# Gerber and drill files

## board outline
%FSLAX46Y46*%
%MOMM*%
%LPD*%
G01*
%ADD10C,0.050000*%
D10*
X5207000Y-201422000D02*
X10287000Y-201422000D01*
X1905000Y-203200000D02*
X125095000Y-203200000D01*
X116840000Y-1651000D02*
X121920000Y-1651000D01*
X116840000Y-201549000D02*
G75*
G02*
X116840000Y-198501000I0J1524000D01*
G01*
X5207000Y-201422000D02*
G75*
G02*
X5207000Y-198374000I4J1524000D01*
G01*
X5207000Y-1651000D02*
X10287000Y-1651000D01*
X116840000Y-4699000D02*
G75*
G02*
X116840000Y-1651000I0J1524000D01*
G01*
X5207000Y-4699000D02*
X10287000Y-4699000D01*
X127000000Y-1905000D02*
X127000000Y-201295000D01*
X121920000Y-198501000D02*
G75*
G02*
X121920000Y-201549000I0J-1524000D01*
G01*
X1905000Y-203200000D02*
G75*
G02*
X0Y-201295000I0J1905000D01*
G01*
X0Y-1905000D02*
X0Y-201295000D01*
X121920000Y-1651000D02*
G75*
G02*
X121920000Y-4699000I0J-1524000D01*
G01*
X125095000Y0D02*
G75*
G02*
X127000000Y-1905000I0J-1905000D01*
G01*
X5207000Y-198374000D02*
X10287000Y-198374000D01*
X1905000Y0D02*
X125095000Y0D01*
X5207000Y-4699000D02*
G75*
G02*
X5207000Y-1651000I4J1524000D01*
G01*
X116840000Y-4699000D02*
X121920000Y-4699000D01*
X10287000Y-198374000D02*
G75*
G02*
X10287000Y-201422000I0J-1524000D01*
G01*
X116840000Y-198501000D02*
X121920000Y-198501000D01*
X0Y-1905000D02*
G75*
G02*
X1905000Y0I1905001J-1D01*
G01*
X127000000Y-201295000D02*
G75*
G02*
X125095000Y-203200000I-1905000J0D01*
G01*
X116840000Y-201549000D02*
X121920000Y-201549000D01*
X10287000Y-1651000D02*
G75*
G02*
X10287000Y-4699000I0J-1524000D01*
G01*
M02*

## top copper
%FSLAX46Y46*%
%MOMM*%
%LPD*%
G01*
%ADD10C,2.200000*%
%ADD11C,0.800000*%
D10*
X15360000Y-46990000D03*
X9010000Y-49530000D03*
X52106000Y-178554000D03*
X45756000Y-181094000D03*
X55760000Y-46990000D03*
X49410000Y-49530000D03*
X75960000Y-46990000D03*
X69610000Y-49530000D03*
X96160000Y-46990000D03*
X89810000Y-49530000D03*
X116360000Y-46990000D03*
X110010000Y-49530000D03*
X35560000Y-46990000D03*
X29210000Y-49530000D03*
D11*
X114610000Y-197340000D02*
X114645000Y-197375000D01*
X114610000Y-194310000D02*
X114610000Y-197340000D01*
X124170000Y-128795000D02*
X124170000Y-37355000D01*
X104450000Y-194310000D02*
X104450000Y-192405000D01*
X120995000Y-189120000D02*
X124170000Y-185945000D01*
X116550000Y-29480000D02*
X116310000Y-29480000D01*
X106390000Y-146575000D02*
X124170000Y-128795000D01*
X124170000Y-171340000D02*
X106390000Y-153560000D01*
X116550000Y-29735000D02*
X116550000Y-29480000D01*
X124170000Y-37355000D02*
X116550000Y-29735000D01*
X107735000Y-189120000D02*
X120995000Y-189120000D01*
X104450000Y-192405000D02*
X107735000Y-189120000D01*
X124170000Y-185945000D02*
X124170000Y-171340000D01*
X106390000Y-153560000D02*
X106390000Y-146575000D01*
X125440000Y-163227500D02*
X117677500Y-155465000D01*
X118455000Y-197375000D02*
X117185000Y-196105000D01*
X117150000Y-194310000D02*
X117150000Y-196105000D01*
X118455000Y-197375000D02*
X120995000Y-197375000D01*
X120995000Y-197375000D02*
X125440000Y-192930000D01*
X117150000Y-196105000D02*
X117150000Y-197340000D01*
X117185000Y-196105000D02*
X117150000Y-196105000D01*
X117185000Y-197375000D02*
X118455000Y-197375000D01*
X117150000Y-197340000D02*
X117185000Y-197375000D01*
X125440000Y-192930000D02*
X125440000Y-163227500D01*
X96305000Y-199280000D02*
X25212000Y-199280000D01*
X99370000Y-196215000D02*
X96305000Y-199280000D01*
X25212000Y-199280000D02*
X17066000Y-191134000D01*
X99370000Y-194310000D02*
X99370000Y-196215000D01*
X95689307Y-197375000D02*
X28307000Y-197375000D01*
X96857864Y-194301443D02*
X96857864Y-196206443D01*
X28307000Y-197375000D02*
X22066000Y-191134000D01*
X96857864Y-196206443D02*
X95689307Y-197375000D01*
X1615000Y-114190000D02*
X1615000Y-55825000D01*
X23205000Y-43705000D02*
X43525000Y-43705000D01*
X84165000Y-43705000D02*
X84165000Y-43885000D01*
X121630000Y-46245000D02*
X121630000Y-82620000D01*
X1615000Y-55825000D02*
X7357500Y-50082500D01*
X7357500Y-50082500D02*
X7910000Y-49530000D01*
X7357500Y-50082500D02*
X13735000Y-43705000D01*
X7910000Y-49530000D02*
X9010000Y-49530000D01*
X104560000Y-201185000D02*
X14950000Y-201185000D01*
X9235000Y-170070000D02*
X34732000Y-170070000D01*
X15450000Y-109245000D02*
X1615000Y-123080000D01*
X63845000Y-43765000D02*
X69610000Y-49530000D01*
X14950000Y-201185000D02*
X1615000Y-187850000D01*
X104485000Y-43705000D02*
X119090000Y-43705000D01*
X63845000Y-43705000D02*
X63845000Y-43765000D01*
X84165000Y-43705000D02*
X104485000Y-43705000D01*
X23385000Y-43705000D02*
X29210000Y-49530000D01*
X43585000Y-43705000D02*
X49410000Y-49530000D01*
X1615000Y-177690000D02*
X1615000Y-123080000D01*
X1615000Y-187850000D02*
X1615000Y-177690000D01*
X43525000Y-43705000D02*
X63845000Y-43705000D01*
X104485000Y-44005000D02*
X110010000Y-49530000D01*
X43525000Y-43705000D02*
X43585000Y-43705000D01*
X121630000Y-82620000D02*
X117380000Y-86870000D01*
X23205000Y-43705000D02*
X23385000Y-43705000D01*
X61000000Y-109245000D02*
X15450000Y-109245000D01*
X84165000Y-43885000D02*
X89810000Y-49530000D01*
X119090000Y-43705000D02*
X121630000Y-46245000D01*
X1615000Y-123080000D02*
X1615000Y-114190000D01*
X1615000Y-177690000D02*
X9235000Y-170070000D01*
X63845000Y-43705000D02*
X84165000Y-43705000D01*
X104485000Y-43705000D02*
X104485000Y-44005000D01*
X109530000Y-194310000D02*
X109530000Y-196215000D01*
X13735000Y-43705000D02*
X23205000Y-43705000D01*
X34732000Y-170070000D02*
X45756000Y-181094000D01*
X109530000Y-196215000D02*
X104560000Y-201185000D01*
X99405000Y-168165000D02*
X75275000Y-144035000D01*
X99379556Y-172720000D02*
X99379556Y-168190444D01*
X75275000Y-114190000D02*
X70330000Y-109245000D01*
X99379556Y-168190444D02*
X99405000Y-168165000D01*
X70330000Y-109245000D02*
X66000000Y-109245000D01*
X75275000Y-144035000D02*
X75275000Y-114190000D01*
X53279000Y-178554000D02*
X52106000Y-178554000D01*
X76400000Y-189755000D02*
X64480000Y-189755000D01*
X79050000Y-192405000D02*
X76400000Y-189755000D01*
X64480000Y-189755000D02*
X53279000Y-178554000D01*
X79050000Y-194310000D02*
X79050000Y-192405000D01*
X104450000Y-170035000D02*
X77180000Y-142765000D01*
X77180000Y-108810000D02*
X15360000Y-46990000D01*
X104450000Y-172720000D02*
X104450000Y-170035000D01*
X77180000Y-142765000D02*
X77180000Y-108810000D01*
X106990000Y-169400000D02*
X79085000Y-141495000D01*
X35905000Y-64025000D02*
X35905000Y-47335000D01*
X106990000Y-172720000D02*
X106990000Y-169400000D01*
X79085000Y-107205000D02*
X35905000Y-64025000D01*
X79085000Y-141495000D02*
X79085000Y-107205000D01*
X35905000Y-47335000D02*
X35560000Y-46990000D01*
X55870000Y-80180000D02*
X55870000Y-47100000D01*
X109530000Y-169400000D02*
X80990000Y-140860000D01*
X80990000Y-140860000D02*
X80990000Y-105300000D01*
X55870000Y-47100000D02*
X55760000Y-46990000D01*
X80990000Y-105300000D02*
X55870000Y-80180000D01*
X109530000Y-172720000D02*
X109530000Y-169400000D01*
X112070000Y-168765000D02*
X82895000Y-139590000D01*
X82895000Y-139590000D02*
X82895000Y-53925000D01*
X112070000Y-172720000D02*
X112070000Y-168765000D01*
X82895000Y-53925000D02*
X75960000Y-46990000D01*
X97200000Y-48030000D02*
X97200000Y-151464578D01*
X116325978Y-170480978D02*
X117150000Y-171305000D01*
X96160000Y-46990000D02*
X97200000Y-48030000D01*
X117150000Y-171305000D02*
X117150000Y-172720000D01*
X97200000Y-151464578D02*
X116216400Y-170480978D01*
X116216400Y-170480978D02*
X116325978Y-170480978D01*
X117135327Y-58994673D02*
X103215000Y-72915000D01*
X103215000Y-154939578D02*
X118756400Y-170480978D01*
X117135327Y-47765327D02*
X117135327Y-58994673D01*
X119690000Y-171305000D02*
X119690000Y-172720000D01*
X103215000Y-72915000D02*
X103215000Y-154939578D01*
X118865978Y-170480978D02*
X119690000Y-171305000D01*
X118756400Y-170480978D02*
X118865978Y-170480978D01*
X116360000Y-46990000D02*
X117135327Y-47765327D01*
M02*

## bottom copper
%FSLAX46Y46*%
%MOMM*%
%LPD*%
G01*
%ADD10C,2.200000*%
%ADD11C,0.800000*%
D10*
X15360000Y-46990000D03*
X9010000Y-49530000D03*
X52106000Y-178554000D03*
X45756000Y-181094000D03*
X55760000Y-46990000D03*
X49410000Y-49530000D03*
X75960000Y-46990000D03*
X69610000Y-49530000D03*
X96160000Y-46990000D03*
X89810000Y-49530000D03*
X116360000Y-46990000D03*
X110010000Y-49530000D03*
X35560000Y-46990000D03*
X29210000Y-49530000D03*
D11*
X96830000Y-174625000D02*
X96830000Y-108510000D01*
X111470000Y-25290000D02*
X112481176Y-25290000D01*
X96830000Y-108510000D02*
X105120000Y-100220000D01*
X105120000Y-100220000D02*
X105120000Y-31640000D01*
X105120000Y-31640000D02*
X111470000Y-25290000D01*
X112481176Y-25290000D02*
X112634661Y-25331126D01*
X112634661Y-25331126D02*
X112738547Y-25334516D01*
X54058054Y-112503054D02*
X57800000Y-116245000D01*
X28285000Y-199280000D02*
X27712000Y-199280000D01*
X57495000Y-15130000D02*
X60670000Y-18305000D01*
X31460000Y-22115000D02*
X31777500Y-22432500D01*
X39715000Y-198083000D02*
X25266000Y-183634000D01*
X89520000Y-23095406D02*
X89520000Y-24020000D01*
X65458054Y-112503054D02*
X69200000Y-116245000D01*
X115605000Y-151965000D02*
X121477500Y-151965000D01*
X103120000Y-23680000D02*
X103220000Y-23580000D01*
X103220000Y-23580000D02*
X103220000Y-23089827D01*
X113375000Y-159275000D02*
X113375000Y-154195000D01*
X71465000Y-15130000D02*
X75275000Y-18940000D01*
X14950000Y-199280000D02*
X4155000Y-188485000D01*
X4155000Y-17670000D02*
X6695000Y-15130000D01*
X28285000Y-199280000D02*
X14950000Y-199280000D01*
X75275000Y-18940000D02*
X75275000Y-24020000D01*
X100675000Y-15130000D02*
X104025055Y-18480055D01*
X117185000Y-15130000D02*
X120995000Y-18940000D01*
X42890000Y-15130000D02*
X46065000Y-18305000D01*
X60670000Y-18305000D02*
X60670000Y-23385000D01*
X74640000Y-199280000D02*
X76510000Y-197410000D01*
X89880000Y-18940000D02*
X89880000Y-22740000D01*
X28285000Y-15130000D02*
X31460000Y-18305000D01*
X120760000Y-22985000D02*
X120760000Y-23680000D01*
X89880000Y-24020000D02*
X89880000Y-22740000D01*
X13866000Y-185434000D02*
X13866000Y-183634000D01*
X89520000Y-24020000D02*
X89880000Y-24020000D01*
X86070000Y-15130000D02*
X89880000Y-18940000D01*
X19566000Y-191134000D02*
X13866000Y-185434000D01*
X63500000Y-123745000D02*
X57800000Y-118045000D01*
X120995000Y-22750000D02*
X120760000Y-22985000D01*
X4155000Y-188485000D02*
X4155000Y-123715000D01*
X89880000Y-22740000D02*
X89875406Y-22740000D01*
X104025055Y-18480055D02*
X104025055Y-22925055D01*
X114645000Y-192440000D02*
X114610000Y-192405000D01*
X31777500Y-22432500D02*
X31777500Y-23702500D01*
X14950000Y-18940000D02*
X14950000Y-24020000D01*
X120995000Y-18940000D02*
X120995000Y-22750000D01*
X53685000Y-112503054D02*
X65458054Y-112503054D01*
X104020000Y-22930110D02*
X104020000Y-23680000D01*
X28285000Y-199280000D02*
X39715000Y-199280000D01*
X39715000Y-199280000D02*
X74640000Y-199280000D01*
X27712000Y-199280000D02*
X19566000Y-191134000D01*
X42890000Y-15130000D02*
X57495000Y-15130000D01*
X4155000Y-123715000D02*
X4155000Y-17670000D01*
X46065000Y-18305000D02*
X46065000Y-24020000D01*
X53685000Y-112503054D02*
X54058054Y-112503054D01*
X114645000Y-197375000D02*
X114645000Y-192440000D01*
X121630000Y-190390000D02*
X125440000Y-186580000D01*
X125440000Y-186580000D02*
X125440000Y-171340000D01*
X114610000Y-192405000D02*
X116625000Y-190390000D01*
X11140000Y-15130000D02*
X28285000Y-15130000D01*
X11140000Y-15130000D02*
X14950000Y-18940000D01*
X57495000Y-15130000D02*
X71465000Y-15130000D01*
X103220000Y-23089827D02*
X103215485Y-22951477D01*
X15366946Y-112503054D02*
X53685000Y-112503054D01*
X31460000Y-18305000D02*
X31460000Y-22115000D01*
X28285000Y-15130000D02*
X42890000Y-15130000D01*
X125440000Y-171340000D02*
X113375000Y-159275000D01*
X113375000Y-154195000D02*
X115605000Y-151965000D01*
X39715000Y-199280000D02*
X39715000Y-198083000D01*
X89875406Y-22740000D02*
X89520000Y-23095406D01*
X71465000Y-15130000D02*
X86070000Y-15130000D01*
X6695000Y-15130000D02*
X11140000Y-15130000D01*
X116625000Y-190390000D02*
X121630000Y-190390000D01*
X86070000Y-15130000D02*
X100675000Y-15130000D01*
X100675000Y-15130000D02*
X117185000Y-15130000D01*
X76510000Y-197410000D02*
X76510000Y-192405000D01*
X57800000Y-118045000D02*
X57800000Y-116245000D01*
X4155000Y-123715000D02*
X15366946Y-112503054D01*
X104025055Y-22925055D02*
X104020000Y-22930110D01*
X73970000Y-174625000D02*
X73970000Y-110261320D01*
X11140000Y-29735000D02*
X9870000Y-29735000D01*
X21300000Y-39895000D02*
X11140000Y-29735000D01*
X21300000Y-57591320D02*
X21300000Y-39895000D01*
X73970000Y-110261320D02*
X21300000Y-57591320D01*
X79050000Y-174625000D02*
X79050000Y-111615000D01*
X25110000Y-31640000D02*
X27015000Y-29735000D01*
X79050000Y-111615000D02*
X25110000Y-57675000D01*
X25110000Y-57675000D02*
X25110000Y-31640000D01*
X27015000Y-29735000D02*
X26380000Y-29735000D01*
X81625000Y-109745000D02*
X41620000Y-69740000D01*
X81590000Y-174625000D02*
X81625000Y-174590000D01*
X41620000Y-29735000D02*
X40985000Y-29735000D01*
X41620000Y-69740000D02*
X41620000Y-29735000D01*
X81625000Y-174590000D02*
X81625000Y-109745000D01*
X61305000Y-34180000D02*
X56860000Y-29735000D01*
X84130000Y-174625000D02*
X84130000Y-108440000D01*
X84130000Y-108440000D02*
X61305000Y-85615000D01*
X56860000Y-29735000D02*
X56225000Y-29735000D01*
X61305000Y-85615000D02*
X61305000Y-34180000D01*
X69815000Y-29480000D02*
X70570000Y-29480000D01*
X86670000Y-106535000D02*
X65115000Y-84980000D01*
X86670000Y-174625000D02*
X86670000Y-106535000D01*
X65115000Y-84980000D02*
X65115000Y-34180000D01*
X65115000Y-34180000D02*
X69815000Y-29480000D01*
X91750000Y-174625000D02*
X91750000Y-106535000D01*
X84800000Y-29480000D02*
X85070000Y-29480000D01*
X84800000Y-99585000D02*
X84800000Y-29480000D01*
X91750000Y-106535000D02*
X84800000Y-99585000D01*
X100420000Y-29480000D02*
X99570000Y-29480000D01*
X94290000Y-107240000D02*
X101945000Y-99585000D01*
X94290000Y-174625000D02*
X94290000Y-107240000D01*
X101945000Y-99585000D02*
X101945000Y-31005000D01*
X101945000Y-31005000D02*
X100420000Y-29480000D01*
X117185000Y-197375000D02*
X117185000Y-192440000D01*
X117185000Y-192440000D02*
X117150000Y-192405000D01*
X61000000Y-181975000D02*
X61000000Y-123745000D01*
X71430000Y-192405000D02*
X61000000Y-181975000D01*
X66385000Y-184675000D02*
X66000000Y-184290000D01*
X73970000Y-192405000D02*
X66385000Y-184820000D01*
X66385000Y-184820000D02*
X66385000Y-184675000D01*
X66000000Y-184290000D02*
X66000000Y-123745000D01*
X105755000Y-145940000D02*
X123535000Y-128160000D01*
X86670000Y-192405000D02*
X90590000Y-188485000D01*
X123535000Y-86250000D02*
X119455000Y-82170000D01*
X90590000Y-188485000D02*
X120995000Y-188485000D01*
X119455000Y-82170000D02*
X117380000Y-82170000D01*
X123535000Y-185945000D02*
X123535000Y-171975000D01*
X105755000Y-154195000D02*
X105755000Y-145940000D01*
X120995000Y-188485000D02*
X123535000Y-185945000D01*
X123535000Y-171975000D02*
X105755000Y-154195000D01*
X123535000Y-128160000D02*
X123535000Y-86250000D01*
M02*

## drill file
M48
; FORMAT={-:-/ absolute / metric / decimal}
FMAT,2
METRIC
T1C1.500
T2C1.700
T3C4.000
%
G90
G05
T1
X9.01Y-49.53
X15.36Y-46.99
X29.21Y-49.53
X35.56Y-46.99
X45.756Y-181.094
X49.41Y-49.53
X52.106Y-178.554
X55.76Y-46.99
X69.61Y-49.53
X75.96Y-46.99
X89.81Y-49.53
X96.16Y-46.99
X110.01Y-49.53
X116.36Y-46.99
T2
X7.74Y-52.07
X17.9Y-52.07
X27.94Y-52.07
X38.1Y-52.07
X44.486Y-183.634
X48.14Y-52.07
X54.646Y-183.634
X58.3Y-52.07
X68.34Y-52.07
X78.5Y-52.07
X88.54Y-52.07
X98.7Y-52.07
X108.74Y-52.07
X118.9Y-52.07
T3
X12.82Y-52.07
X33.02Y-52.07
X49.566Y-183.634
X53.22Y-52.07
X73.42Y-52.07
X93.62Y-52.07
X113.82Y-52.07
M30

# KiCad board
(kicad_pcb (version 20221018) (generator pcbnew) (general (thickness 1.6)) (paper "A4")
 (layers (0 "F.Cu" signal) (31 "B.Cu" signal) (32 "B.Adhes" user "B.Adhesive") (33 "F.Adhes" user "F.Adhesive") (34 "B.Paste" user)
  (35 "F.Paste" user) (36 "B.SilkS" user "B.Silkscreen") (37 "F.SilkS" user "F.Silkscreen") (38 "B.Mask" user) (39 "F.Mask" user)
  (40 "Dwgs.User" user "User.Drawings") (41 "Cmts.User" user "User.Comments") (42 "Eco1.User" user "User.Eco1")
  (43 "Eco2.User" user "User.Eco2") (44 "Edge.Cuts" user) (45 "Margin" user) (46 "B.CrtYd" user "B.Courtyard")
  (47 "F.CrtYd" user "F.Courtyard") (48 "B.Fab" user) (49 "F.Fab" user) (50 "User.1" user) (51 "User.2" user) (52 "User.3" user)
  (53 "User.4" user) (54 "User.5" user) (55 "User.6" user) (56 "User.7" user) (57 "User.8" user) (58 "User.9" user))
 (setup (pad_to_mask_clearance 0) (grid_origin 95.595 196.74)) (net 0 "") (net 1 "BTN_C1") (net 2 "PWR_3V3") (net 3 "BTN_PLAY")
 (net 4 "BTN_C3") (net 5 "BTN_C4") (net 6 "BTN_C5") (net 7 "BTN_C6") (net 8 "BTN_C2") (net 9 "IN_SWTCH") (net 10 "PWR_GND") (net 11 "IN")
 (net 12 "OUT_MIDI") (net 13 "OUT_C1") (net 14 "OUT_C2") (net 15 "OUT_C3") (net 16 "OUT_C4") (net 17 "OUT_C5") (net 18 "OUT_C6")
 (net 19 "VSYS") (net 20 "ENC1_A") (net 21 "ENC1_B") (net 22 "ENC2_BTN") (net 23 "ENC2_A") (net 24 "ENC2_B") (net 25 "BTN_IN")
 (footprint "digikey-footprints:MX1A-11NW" (layer "F.Cu") (at 11.55 42.545)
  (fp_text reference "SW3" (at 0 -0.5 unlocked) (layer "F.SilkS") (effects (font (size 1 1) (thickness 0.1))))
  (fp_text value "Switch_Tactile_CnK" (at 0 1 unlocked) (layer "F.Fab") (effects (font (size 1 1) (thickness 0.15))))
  (pad "" np_thru_hole circle (at -3.81 9.525) (size 1.7 1.7) (drill 1.7) (layers "*.Cu" "*.Mask"))
  (pad "" np_thru_hole circle (at 1.27 9.525) (size 4 4) (drill 4) (layers "*.Cu" "*.Mask"))
  (pad "" np_thru_hole circle (at 6.35 9.525) (size 1.7 1.7) (drill 1.7) (layers "*.Cu" "*.Mask"))
  (pad "1" thru_hole circle (at 3.81 4.445) (size 2.2 2.2) (drill 1.5) (layers "*.Cu" "*.Mask") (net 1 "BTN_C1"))
  (pad "2" thru_hole circle (at -2.54 6.985) (size 2.2 2.2) (drill 1.5) (layers "*.Cu" "*.Mask") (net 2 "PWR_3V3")))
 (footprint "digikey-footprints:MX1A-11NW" (layer "F.Cu") (at 48.296 174.109)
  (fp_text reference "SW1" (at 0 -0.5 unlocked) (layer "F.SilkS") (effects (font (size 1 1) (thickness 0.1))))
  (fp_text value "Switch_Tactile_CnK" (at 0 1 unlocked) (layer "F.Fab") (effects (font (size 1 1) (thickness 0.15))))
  (pad "" np_thru_hole circle (at -3.81 9.525) (size 1.7 1.7) (drill 1.7) (layers "*.Cu" "*.Mask"))
  (pad "" np_thru_hole circle (at 1.27 9.525) (size 4 4) (drill 4) (layers "*.Cu" "*.Mask"))
  (pad "" np_thru_hole circle (at 6.35 9.525) (size 1.7 1.7) (drill 1.7) (layers "*.Cu" "*.Mask"))
  (pad "1" thru_hole circle (at 3.81 4.445) (size 2.2 2.2) (drill 1.5) (layers "*.Cu" "*.Mask") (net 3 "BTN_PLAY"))
  (pad "2" thru_hole circle (at -2.54 6.985) (size 2.2 2.2) (drill 1.5) (layers "*.Cu" "*.Mask") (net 2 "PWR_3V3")))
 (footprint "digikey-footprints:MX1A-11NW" (layer "F.Cu") (at 51.95 42.545)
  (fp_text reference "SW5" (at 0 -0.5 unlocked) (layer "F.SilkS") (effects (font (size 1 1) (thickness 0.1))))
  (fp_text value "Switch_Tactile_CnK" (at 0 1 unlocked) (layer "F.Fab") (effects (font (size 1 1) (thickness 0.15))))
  (pad "" np_thru_hole circle (at -3.81 9.525) (size 1.7 1.7) (drill 1.7) (layers "*.Cu" "*.Mask"))
  (pad "" np_thru_hole circle (at 1.27 9.525) (size 4 4) (drill 4) (layers "*.Cu" "*.Mask"))
  (pad "" np_thru_hole circle (at 6.35 9.525) (size 1.7 1.7) (drill 1.7) (layers "*.Cu" "*.Mask"))
  (pad "1" thru_hole circle (at 3.81 4.445) (size 2.2 2.2) (drill 1.5) (layers "*.Cu" "*.Mask") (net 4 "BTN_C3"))
  (pad "2" thru_hole circle (at -2.54 6.985) (size 2.2 2.2) (drill 1.5) (layers "*.Cu" "*.Mask") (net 2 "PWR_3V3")))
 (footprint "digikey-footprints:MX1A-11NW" (layer "F.Cu") (at 72.15 42.545)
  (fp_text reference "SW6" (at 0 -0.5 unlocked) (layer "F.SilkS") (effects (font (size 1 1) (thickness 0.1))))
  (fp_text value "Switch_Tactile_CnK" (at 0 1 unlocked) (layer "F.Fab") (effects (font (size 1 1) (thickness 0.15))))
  (pad "" np_thru_hole circle (at -3.81 9.525) (size 1.7 1.7) (drill 1.7) (layers "*.Cu" "*.Mask"))
  (pad "" np_thru_hole circle (at 1.27 9.525) (size 4 4) (drill 4) (layers "*.Cu" "*.Mask"))
  (pad "" np_thru_hole circle (at 6.35 9.525) (size 1.7 1.7) (drill 1.7) (layers "*.Cu" "*.Mask"))
  (pad "1" thru_hole circle (at 3.81 4.445) (size 2.2 2.2) (drill 1.5) (layers "*.Cu" "*.Mask") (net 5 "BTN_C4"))
  (pad "2" thru_hole circle (at -2.54 6.985) (size 2.2 2.2) (drill 1.5) (layers "*.Cu" "*.Mask") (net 2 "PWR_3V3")))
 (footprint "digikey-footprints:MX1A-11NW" (layer "F.Cu") (at 92.35 42.545)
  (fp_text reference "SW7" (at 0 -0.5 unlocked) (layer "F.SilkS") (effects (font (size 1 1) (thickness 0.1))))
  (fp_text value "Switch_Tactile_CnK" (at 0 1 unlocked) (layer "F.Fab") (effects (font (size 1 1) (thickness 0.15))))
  (pad "" np_thru_hole circle (at -3.81 9.525) (size 1.7 1.7) (drill 1.7) (layers "*.Cu" "*.Mask"))
  (pad "" np_thru_hole circle (at 1.27 9.525) (size 4 4) (drill 4) (layers "*.Cu" "*.Mask"))
  (pad "" np_thru_hole circle (at 6.35 9.525) (size 1.7 1.7) (drill 1.7) (layers "*.Cu" "*.Mask"))
  (pad "1" thru_hole circle (at 3.81 4.445) (size 2.2 2.2) (drill 1.5) (layers "*.Cu" "*.Mask") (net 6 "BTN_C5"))
  (pad "2" thru_hole circle (at -2.54 6.985) (size 2.2 2.2) (drill 1.5) (layers "*.Cu" "*.Mask") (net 2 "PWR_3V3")))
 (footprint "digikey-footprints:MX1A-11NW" (layer "F.Cu") (at 112.55 42.545)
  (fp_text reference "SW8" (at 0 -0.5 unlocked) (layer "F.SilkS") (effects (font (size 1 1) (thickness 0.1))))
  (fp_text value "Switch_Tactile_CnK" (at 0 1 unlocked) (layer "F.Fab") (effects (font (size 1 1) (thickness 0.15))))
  (pad "" np_thru_hole circle (at -3.81 9.525) (size 1.7 1.7) (drill 1.7) (layers "*.Cu" "*.Mask"))
  (pad "" np_thru_hole circle (at 1.27 9.525) (size 4 4) (drill 4) (layers "*.Cu" "*.Mask"))
  (pad "" np_thru_hole circle (at 6.35 9.525) (size 1.7 1.7) (drill 1.7) (layers "*.Cu" "*.Mask"))
  (pad "1" thru_hole circle (at 3.81 4.445) (size 2.2 2.2) (drill 1.5) (layers "*.Cu" "*.Mask") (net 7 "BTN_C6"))
  (pad "2" thru_hole circle (at -2.54 6.985) (size 2.2 2.2) (drill 1.5) (layers "*.Cu" "*.Mask") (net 2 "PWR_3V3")))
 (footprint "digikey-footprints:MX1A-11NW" (layer "F.Cu") (at 31.75 42.545)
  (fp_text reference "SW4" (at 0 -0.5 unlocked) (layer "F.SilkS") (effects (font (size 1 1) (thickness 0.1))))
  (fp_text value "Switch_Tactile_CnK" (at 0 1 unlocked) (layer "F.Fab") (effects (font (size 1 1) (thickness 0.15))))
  (pad "" np_thru_hole circle (at -3.81 9.525) (size 1.7 1.7) (drill 1.7) (layers "*.Cu" "*.Mask"))
  (pad "" np_thru_hole circle (at 1.27 9.525) (size 4 4) (drill 4) (layers "*.Cu" "*.Mask"))
  (pad "" np_thru_hole circle (at 6.35 9.525) (size 1.7 1.7) (drill 1.7) (layers "*.Cu" "*.Mask"))
  (pad "1" thru_hole circle (at 3.81 4.445) (size 2.2 2.2) (drill 1.5) (layers "*.Cu" "*.Mask") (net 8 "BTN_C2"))
  (pad "2" thru_hole circle (at -2.54 6.985) (size 2.2 2.2) (drill 1.5) (layers "*.Cu" "*.Mask") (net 2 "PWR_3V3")))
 (gr_line (start 5.207 201.422) (end 10.287 201.422) (stroke (width 0.05) (type solid)) (layer "Edge.Cuts"))
 (gr_line (start 1.905 203.2) (end 125.095 203.2) (stroke (width 0.05) (type default)) (layer "Edge.Cuts"))
 (gr_line (start 116.84 1.651) (end 121.92 1.651) (stroke (width 0.05) (type solid)) (layer "Edge.Cuts"))
 (gr_arc (start 116.84 201.549) (mid 115.316004 200.025002) (end 116.84 198.501) (stroke (width 0.05) (type solid)) (layer "Edge.Cuts"))
 (gr_arc (start 5.207 201.422) (mid 3.683004 199.898002) (end 5.207 198.374) (stroke (width 0.05) (type solid)) (layer "Edge.Cuts"))
 (gr_line (start 5.207 1.651) (end 10.287 1.651) (stroke (width 0.05) (type solid)) (layer "Edge.Cuts"))
 (gr_arc (start 116.84 4.699) (mid 115.316004 3.175002) (end 116.84 1.651) (stroke (width 0.05) (type solid)) (layer "Edge.Cuts"))
 (gr_line (start 5.207 4.699) (end 10.287 4.699) (stroke (width 0.05) (type solid)) (layer "Edge.Cuts"))
 (gr_line (start 127 1.905) (end 127 201.295) (stroke (width 0.05) (type default)) (layer "Edge.Cuts"))
 (gr_arc (start 121.92 198.501) (mid 123.444004 200.025002) (end 121.92 201.549) (stroke (width 0.05) (type solid)) (layer "Edge.Cuts"))
 (gr_arc (start 1.905 203.2) (mid 0.557962 202.642038) (end 0 201.295) (stroke (width 0.05) (type solid)) (layer "Edge.Cuts"))
 (gr_line (start 0 1.905) (end 0 201.295) (stroke (width 0.05) (type default)) (layer "Edge.Cuts"))
 (gr_arc (start 121.92 1.651) (mid 123.444004 3.175002) (end 121.92 4.699) (stroke (width 0.05) (type solid)) (layer "Edge.Cuts"))
 (gr_arc (start 125.095 0) (mid 126.442038 0.557962) (end 127 1.905) (stroke (width 0.05) (type solid)) (layer "Edge.Cuts"))
 (gr_line (start 5.207 198.374) (end 10.287 198.374) (stroke (width 0.05) (type solid)) (layer "Edge.Cuts"))
 (gr_line (start 1.905 0) (end 125.095 0) (stroke (width 0.05) (type default)) (layer "Edge.Cuts"))
 (gr_arc (start 5.207 4.699) (mid 3.683004 3.175002) (end 5.207 1.651) (stroke (width 0.05) (type solid)) (layer "Edge.Cuts"))
 (gr_line (start 116.84 4.699) (end 121.92 4.699) (stroke (width 0.05) (type solid)) (layer "Edge.Cuts"))
 (gr_arc (start 10.287 198.374) (mid 11.811004 199.898002) (end 10.287 201.422) (stroke (width 0.05) (type solid)) (layer "Edge.Cuts"))
 (gr_line (start 116.84 198.501) (end 121.92 198.501) (stroke (width 0.05) (type solid)) (layer "Edge.Cuts"))
 (gr_arc (start 0 1.905) (mid 0.557962 0.557962) (end 1.905 0) (stroke (width 0.05) (type solid)) (layer "Edge.Cuts"))
 (gr_arc (start 127 201.295) (mid 126.442038 202.642038) (end 125.095 203.2) (stroke (width 0.05) (type solid)) (layer "Edge.Cuts"))
 (gr_line (start 116.84 201.549) (end 121.92 201.549) (stroke (width 0.05) (type solid)) (layer "Edge.Cuts"))
 (gr_arc (start 10.287 1.651) (mid 11.811004 3.175002) (end 10.287 4.699) (stroke (width 0.05) (type solid)) (layer "Edge.Cuts"))
 (segment (start 96.83 174.625) (end 96.83 108.51) (width 0.8) (layer "B.Cu") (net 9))
 (segment (start 111.47 25.29) (end 112.481176 25.29) (width 0.8) (layer "B.Cu") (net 9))
 (segment (start 96.83 108.51) (end 105.12 100.22) (width 0.8) (layer "B.Cu") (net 9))
 (segment (start 105.12 100.22) (end 105.12 31.64) (width 0.8) (layer "B.Cu") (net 9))
 (segment (start 105.12 31.64) (end 111.47 25.29) (width 0.8) (layer "B.Cu") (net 9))
 (segment (start 112.481176 25.29) (end 112.634661 25.331126) (width 0.8) (layer "B.Cu") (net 9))
 (segment (start 112.634661 25.331126) (end 112.738547 25.334516) (width 0.8) (layer "B.Cu") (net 9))
 (segment (start 114.61 197.34) (end 114.645 197.375) (width 0.8) (layer "F.Cu") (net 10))
 (segment (start 114.61 194.31) (end 114.61 197.34) (width 0.8) (layer "F.Cu") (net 10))
 (segment (start 54.058054 112.503054) (end 57.8 116.245) (width 0.8) (layer "B.Cu") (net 10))
 (segment (start 28.285 199.28) (end 27.712 199.28) (width 0.8) (layer "B.Cu") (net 10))
 (segment (start 57.495 15.13) (end 60.67 18.305) (width 0.8) (layer "B.Cu") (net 10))
 (segment (start 31.46 22.115) (end 31.7775 22.4325) (width 0.8) (layer "B.Cu") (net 10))
 (segment (start 39.715 198.083) (end 25.266 183.634) (width 0.8) (layer "B.Cu") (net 10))
 (segment (start 89.52 23.095406) (end 89.52 24.02) (width 0.8) (layer "B.Cu") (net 10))
 (segment (start 65.458054 112.503054) (end 69.2 116.245) (width 0.8) (layer "B.Cu") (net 10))
 (segment (start 115.605 151.965) (end 121.4775 151.965) (width 0.8) (layer "B.Cu") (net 10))
 (segment (start 103.12 23.68) (end 103.22 23.58) (width 0.8) (layer "B.Cu") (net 10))
 (segment (start 103.22 23.58) (end 103.22 23.089827) (width 0.8) (layer "B.Cu") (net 10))
 (segment (start 113.375 159.275) (end 113.375 154.195) (width 0.8) (layer "B.Cu") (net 10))
 (segment (start 71.465 15.13) (end 75.275 18.94) (width 0.8) (layer "B.Cu") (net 10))
 (segment (start 14.95 199.28) (end 4.155 188.485) (width 0.8) (layer "B.Cu") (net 10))
 (segment (start 4.155 17.67) (end 6.695 15.13) (width 0.8) (layer "B.Cu") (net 10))
 (segment (start 28.285 199.28) (end 14.95 199.28) (width 0.8) (layer "B.Cu") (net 10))
 (segment (start 75.275 18.94) (end 75.275 24.02) (width 0.8) (layer "B.Cu") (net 10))
 (segment (start 100.675 15.13) (end 104.025055 18.480055) (width 0.8) (layer "B.Cu") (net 10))
 (segment (start 117.185 15.13) (end 120.995 18.94) (width 0.8) (layer "B.Cu") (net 10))
 (segment (start 42.89 15.13) (end 46.065 18.305) (width 0.8) (layer "B.Cu") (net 10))
 (segment (start 60.67 18.305) (end 60.67 23.385) (width 0.8) (layer "B.Cu") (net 10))
 (segment (start 74.64 199.28) (end 76.51 197.41) (width 0.8) (layer "B.Cu") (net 10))
 (segment (start 89.88 18.94) (end 89.88 22.74) (width 0.8) (layer "B.Cu") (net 10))
 (segment (start 28.285 15.13) (end 31.46 18.305) (width 0.8) (layer "B.Cu") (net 10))
 (segment (start 120.76 22.985) (end 120.76 23.68) (width 0.8) (layer "B.Cu") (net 10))
 (segment (start 89.88 24.02) (end 89.88 22.74) (width 0.8) (layer "B.Cu") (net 10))
 (segment (start 13.866 185.434) (end 13.866 183.634) (width 0.8) (layer "B.Cu") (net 10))
 (segment (start 89.52 24.02) (end 89.88 24.02) (width 0.8) (layer "B.Cu") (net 10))
 (segment (start 86.07 15.13) (end 89.88 18.94) (width 0.8) (layer "B.Cu") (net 10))
 (segment (start 19.566 191.134) (end 13.866 185.434) (width 0.8) (layer "B.Cu") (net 10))
 (segment (start 63.5 123.745) (end 57.8 118.045) (width 0.8) (layer "B.Cu") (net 10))
 (segment (start 120.995 22.75) (end 120.76 22.985) (width 0.8) (layer "B.Cu") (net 10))
 (segment (start 4.155 188.485) (end 4.155 123.715) (width 0.8) (layer "B.Cu") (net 10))
 (segment (start 89.88 22.74) (end 89.875406 22.74) (width 0.8) (layer "B.Cu") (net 10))
 (segment (start 104.025055 18.480055) (end 104.025055 22.925055) (width 0.8) (layer "B.Cu") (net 10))
 (segment (start 114.645 192.44) (end 114.61 192.405) (width 0.8) (layer "B.Cu") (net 10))
 (segment (start 31.7775 22.4325) (end 31.7775 23.7025) (width 0.8) (layer "B.Cu") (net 10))
 (segment (start 14.95 18.94) (end 14.95 24.02) (width 0.8) (layer "B.Cu") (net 10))
 (segment (start 120.995 18.94) (end 120.995 22.75) (width 0.8) (layer "B.Cu") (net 10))
 (segment (start 53.685 112.503054) (end 65.458054 112.503054) (width 0.8) (layer "B.Cu") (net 10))
 (segment (start 104.02 22.93011) (end 104.02 23.68) (width 0.8) (layer "B.Cu") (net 10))
 (segment (start 28.285 199.28) (end 39.715 199.28) (width 0.8) (layer "B.Cu") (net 10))
 (segment (start 39.715 199.28) (end 74.64 199.28) (width 0.8) (layer "B.Cu") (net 10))
 (segment (start 27.712 199.28) (end 19.566 191.134) (width 0.8) (layer "B.Cu") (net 10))
 (segment (start 42.89 15.13) (end 57.495 15.13) (width 0.8) (layer "B.Cu") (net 10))
 (segment (start 4.155 123.715) (end 4.155 17.67) (width 0.8) (layer "B.Cu") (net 10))
 (segment (start 46.065 18.305) (end 46.065 24.02) (width 0.8) (layer "B.Cu") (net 10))
 (segment (start 53.685 112.503054) (end 54.058054 112.503054) (width 0.8) (layer "B.Cu") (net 10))
 (segment (start 114.645 197.375) (end 114.645 192.44) (width 0.8) (layer "B.Cu") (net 10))
 (segment (start 121.63 190.39) (end 125.44 186.58) (width 0.8) (layer "B.Cu") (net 10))
 (segment (start 125.44 186.58) (end 125.44 171.34) (width 0.8) (layer "B.Cu") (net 10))
 (segment (start 114.61 192.405) (end 116.625 190.39) (width 0.8) (layer "B.Cu") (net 10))
 (segment (start 11.14 15.13) (end 28.285 15.13) (width 0.8) (layer "B.Cu") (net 10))
 (segment (start 11.14 15.13) (end 14.95 18.94) (width 0.8) (layer "B.Cu") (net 10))
 (segment (start 57.495 15.13) (end 71.465 15.13) (width 0.8) (layer "B.Cu") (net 10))
 (segment (start 103.22 23.089827) (end 103.215485 22.951477) (width 0.8) (layer "B.Cu") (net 10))
 (segment (start 15.366946 112.503054) (end 53.685 112.503054) (width 0.8) (layer "B.Cu") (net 10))
 (segment (start 31.46 18.305) (end 31.46 22.115) (width 0.8) (layer "B.Cu") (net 10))
 (segment (start 28.285 15.13) (end 42.89 15.13) (width 0.8) (layer "B.Cu") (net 10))
 (segment (start 125.44 171.34) (end 113.375 159.275) (width 0.8) (layer "B.Cu") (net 10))
 (segment (start 113.375 154.195) (end 115.605 151.965) (width 0.8) (layer "B.Cu") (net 10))
 (segment (start 39.715 199.28) (end 39.715 198.083) (width 0.8) (layer "B.Cu") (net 10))
 (segment (start 89.875406 22.74) (end 89.52 23.095406) (width 0.8) (layer "B.Cu") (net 10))
 (segment (start 71.465 15.13) (end 86.07 15.13) (width 0.8) (layer "B.Cu") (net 10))
 (segment (start 6.695 15.13) (end 11.14 15.13) (width 0.8) (layer "B.Cu") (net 10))
 (segment (start 116.625 190.39) (end 121.63 190.39) (width 0.8) (layer "B.Cu") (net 10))
 (segment (start 86.07 15.13) (end 100.675 15.13) (width 0.8) (layer "B.Cu") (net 10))
 (segment (start 100.675 15.13) (end 117.185 15.13) (width 0.8) (layer "B.Cu") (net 10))
 (segment (start 76.51 197.41) (end 76.51 192.405) (width 0.8) (layer "B.Cu") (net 10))
 (segment (start 57.8 118.045) (end 57.8 116.245) (width 0.8) (layer "B.Cu") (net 10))
 (segment (start 4.155 123.715) (end 15.366946 112.503054) (width 0.8) (layer "B.Cu") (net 10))
 (segment (start 104.025055 22.925055) (end 104.02 22.93011) (width 0.8) (layer "B.Cu") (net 10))
 (segment (start 124.17 128.795) (end 124.17 37.355) (width 0.8) (layer "F.Cu") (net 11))
 (segment (start 104.45 194.31) (end 104.45 192.405) (width 0.8) (layer "F.Cu") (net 11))
 (segment (start 120.995 189.12) (end 124.17 185.945) (width 0.8) (layer "F.Cu") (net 11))
 (segment (start 116.55 29.48) (end 116.31 29.48) (width 0.8) (layer "F.Cu") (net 11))
 (segment (start 106.39 146.575) (end 124.17 128.795) (width 0.8) (layer "F.Cu") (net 11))
 (segment (start 124.17 171.34) (end 106.39 153.56) (width 0.8) (layer "F.Cu") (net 11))
 (segment (start 116.55 29.735) (end 116.55 29.48) (width 0.8) (layer "F.Cu") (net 11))
 (segment (start 124.17 37.355) (end 116.55 29.735) (width 0.8) (layer "F.Cu") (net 11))
 (segment (start 107.735 189.12) (end 120.995 189.12) (width 0.8) (layer "F.Cu") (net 11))
 (segment (start 104.45 192.405) (end 107.735 189.12) (width 0.8) (layer "F.Cu") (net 11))
 (segment (start 124.17 185.945) (end 124.17 171.34) (width 0.8) (layer "F.Cu") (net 11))
 (segment (start 106.39 153.56) (end 106.39 146.575) (width 0.8) (layer "F.Cu") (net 11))
 (segment (start 73.97 174.625) (end 73.97 110.26132) (width 0.8) (layer "B.Cu") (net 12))
 (segment (start 11.14 29.735) (end 9.87 29.735) (width 0.8) (layer "B.Cu") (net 12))
 (segment (start 21.3 39.895) (end 11.14 29.735) (width 0.8) (layer "B.Cu") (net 12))
 (segment (start 21.3 57.59132) (end 21.3 39.895) (width 0.8) (layer "B.Cu") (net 12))
 (segment (start 73.97 110.26132) (end 21.3 57.59132) (width 0.8) (layer "B.Cu") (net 12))
 (segment (start 79.05 174.625) (end 79.05 111.615) (width 0.8) (layer "B.Cu") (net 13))
 (segment (start 25.11 31.64) (end 27.015 29.735) (width 0.8) (layer "B.Cu") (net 13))
 (segment (start 79.05 111.615) (end 25.11 57.675) (width 0.8) (layer "B.Cu") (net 13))
 (segment (start 25.11 57.675) (end 25.11 31.64) (width 0.8) (layer "B.Cu") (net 13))
 (segment (start 27.015 29.735) (end 26.38 29.735) (width 0.8) (layer "B.Cu") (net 13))
 (segment (start 81.625 109.745) (end 41.62 69.74) (width 0.8) (layer "B.Cu") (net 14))
 (segment (start 81.59 174.625) (end 81.625 174.59) (width 0.8) (layer "B.Cu") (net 14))
 (segment (start 41.62 29.735) (end 40.985 29.735) (width 0.8) (layer "B.Cu") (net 14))
 (segment (start 41.62 69.74) (end 41.62 29.735) (width 0.8) (layer "B.Cu") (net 14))
 (segment (start 81.625 174.59) (end 81.625 109.745) (width 0.8) (layer "B.Cu") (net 14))
 (segment (start 61.305 34.18) (end 56.86 29.735) (width 0.8) (layer "B.Cu") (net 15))
 (segment (start 84.13 174.625) (end 84.13 108.44) (width 0.8) (layer "B.Cu") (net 15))
 (segment (start 84.13 108.44) (end 61.305 85.615) (width 0.8) (layer "B.Cu") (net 15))
 (segment (start 56.86 29.735) (end 56.225 29.735) (width 0.8) (layer "B.Cu") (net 15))
 (segment (start 61.305 85.615) (end 61.305 34.18) (width 0.8) (layer "B.Cu") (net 15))
 (segment (start 69.815 29.48) (end 70.57 29.48) (width 0.8) (layer "B.Cu") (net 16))
 (segment (start 86.67 106.535) (end 65.115 84.98) (width 0.8) (layer "B.Cu") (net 16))
 (segment (start 86.67 174.625) (end 86.67 106.535) (width 0.8) (layer "B.Cu") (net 16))
 (segment (start 65.115 84.98) (end 65.115 34.18) (width 0.8) (layer "B.Cu") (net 16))
 (segment (start 65.115 34.18) (end 69.815 29.48) (width 0.8) (layer "B.Cu") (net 16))
 (segment (start 91.75 174.625) (end 91.75 106.535) (width 0.8) (layer "B.Cu") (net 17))
 (segment (start 84.8 29.48) (end 85.07 29.48) (width 0.8) (layer "B.Cu") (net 17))
 (segment (start 84.8 99.585) (end 84.8 29.48) (width 0.8) (layer "B.Cu") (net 17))
 (segment (start 91.75 106.535) (end 84.8 99.585) (width 0.8) (layer "B.Cu") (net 17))
 (segment (start 100.42 29.48) (end 99.57 29.48) (width 0.8) (layer "B.Cu") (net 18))
 (segment (start 94.29 107.24) (end 101.945 99.585) (width 0.8) (layer "B.Cu") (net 18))
 (segment (start 94.29 174.625) (end 94.29 107.24) (width 0.8) (layer "B.Cu") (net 18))
 (segment (start 101.945 99.585) (end 101.945 31.005) (width 0.8) (layer "B.Cu") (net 18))
 (segment (start 101.945 31.005) (end 100.42 29.48) (width 0.8) (layer "B.Cu") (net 18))
 (segment (start 125.44 163.2275) (end 117.6775 155.465) (width 0.8) (layer "F.Cu") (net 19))
 (segment (start 118.455 197.375) (end 117.185 196.105) (width 0.8) (layer "F.Cu") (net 19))
 (segment (start 117.15 194.31) (end 117.15 196.105) (width 0.8) (layer "F.Cu") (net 19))
 (segment (start 118.455 197.375) (end 120.995 197.375) (width 0.8) (layer "F.Cu") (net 19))
 (segment (start 120.995 197.375) (end 125.44 192.93) (width 0.8) (layer "F.Cu") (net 19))
 (segment (start 117.15 196.105) (end 117.15 197.34) (width 0.8) (layer "F.Cu") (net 19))
 (segment (start 117.185 196.105) (end 117.15 196.105) (width 0.8) (layer "F.Cu") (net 19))
 (segment (start 117.185 197.375) (end 118.455 197.375) (width 0.8) (layer "F.Cu") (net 19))
 (segment (start 117.15 197.34) (end 117.185 197.375) (width 0.8) (layer "F.Cu") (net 19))
 (segment (start 125.44 192.93) (end 125.44 163.2275) (width 0.8) (layer "F.Cu") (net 19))
 (segment (start 117.185 197.375) (end 117.185 192.44) (width 0.8) (layer "B.Cu") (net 19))
 (segment (start 117.185 192.44) (end 117.15 192.405) (width 0.8) (layer "B.Cu") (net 19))
 (segment (start 96.305 199.28) (end 25.212 199.28) (width 0.8) (layer "F.Cu") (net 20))
 (segment (start 99.37 196.215) (end 96.305 199.28) (width 0.8) (layer "F.Cu") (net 20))
 (segment (start 25.212 199.28) (end 17.066 191.134) (width 0.8) (layer "F.Cu") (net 20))
 (segment (start 99.37 194.31) (end 99.37 196.215) (width 0.8) (layer "F.Cu") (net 20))
 (segment (start 95.689307 197.375) (end 28.307 197.375) (width 0.8) (layer "F.Cu") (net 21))
 (segment (start 96.857864 194.301443) (end 96.857864 196.206443) (width 0.8) (layer "F.Cu") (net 21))
 (segment (start 28.307 197.375) (end 22.066 191.134) (width 0.8) (layer "F.Cu") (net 21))
 (segment (start 96.857864 196.206443) (end 95.689307 197.375) (width 0.8) (layer "F.Cu") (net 21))
 (segment (start 1.615 114.19) (end 1.615 55.825) (width 0.8) (layer "F.Cu") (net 2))
 (segment (start 23.205 43.705) (end 43.525 43.705) (width 0.8) (layer "F.Cu") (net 2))
 (segment (start 84.165 43.705) (end 84.165 43.885) (width 0.8) (layer "F.Cu") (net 2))
 (segment (start 121.63 46.245) (end 121.63 82.62) (width 0.8) (layer "F.Cu") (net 2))
 (segment (start 1.615 55.825) (end 7.3575 50.0825) (width 0.8) (layer "F.Cu") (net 2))
 (segment (start 7.3575 50.0825) (end 7.91 49.53) (width 0.8) (layer "F.Cu") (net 2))
 (segment (start 7.3575 50.0825) (end 13.735 43.705) (width 0.8) (layer "F.Cu") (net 2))
 (segment (start 7.91 49.53) (end 9.01 49.53) (width 0.8) (layer "F.Cu") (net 2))
 (segment (start 104.56 201.185) (end 14.95 201.185) (width 0.8) (layer "F.Cu") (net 2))
 (segment (start 9.235 170.07) (end 34.732 170.07) (width 0.8) (layer "F.Cu") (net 2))
 (segment (start 15.45 109.245) (end 1.615 123.08) (width 0.8) (layer "F.Cu") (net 2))
 (segment (start 63.845 43.765) (end 69.61 49.53) (width 0.8) (layer "F.Cu") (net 2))
 (segment (start 14.95 201.185) (end 1.615 187.85) (width 0.8) (layer "F.Cu") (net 2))
 (segment (start 104.485 43.705) (end 119.09 43.705) (width 0.8) (layer "F.Cu") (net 2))
 (segment (start 63.845 43.705) (end 63.845 43.765) (width 0.8) (layer "F.Cu") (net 2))
 (segment (start 84.165 43.705) (end 104.485 43.705) (width 0.8) (layer "F.Cu") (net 2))
 (segment (start 23.385 43.705) (end 29.21 49.53) (width 0.8) (layer "F.Cu") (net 2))
 (segment (start 43.585 43.705) (end 49.41 49.53) (width 0.8) (layer "F.Cu") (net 2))
 (segment (start 1.615 177.69) (end 1.615 123.08) (width 0.8) (layer "F.Cu") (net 2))
 (segment (start 1.615 187.85) (end 1.615 177.69) (width 0.8) (layer "F.Cu") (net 2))
 (segment (start 43.525 43.705) (end 63.845 43.705) (width 0.8) (layer "F.Cu") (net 2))
 (segment (start 104.485 44.005) (end 110.01 49.53) (width 0.8) (layer "F.Cu") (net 2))
 (segment (start 43.525 43.705) (end 43.585 43.705) (width 0.8) (layer "F.Cu") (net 2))
 (segment (start 121.63 82.62) (end 117.38 86.87) (width 0.8) (layer "F.Cu") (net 2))
 (segment (start 23.205 43.705) (end 23.385 43.705) (width 0.8) (layer "F.Cu") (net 2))
 (segment (start 61 109.245) (end 15.45 109.245) (width 0.8) (layer "F.Cu") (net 2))
 (segment (start 84.165 43.885) (end 89.81 49.53) (width 0.8) (layer "F.Cu") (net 2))
 (segment (start 119.09 43.705) (end 121.63 46.245) (width 0.8) (layer "F.Cu") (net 2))
 (segment (start 1.615 123.08) (end 1.615 114.19) (width 0.8) (layer "F.Cu") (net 2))
 (segment (start 1.615 177.69) (end 9.235 170.07) (width 0.8) (layer "F.Cu") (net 2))
 (segment (start 63.845 43.705) (end 84.165 43.705) (width 0.8) (layer "F.Cu") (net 2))
 (segment (start 104.485 43.705) (end 104.485 44.005) (width 0.8) (layer "F.Cu") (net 2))
 (segment (start 109.53 194.31) (end 109.53 196.215) (width 0.8) (layer "F.Cu") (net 2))
 (segment (start 13.735 43.705) (end 23.205 43.705) (width 0.8) (layer "F.Cu") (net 2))
 (segment (start 34.732 170.07) (end 45.756 181.094) (width 0.8) (layer "F.Cu") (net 2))
 (segment (start 109.53 196.215) (end 104.56 201.185) (width 0.8) (layer "F.Cu") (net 2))
 (segment (start 99.405 168.165) (end 75.275 144.035) (width 0.8) (layer "F.Cu") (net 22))
 (segment (start 99.379556 172.72) (end 99.379556 168.190444) (width 0.8) (layer "F.Cu") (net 22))
 (segment (start 75.275 114.19) (end 70.33 109.245) (width 0.8) (layer "F.Cu") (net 22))
 (segment (start 99.379556 168.190444) (end 99.405 168.165) (width 0.8) (layer "F.Cu") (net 22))
 (segment (start 70.33 109.245) (end 66 109.245) (width 0.8) (layer "F.Cu") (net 22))
 (segment (start 75.275 144.035) (end 75.275 114.19) (width 0.8) (layer "F.Cu") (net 22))
 (segment (start 61 181.975) (end 61 123.745) (width 0.8) (layer "B.Cu") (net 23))
 (segment (start 71.43 192.405) (end 61 181.975) (width 0.8) (layer "B.Cu") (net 23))
 (segment (start 66.385 184.675) (end 66 184.29) (width 0.8) (layer "B.Cu") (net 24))
 (segment (start 73.97 192.405) (end 66.385 184.82) (width 0.8) (layer "B.Cu") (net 24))
 (segment (start 66.385 184.82) (end 66.385 184.675) (width 0.8) (layer "B.Cu") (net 24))
 (segment (start 66 184.29) (end 66 123.745) (width 0.8) (layer "B.Cu") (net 24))
 (segment (start 105.755 145.94) (end 123.535 128.16) (width 0.8) (layer "B.Cu") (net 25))
 (segment (start 86.67 192.405) (end 90.59 188.485) (width 0.8) (layer "B.Cu") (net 25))
 (segment (start 123.535 86.25) (end 119.455 82.17) (width 0.8) (layer "B.Cu") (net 25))
 (segment (start 90.59 188.485) (end 120.995 188.485) (width 0.8) (layer "B.Cu") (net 25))
 (segment (start 119.455 82.17) (end 117.38 82.17) (width 0.8) (layer "B.Cu") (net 25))
 (segment (start 123.535 185.945) (end 123.535 171.975) (width 0.8) (layer "B.Cu") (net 25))
 (segment (start 105.755 154.195) (end 105.755 145.94) (width 0.8) (layer "B.Cu") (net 25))
 (segment (start 120.995 188.485) (end 123.535 185.945) (width 0.8) (layer "B.Cu") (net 25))
 (segment (start 123.535 171.975) (end 105.755 154.195) (width 0.8) (layer "B.Cu") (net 25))
 (segment (start 123.535 128.16) (end 123.535 86.25) (width 0.8) (layer "B.Cu") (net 25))
 (segment (start 53.279 178.554) (end 52.106 178.554) (width 0.8) (layer "F.Cu") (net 3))
 (segment (start 76.4 189.755) (end 64.48 189.755) (width 0.8) (layer "F.Cu") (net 3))
 (segment (start 79.05 192.405) (end 76.4 189.755) (width 0.8) (layer "F.Cu") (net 3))
 (segment (start 64.48 189.755) (end 53.279 178.554) (width 0.8) (layer "F.Cu") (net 3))
 (segment (start 79.05 194.31) (end 79.05 192.405) (width 0.8) (layer "F.Cu") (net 3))
 (segment (start 104.45 170.035) (end 77.18 142.765) (width 0.8) (layer "F.Cu") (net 1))
 (segment (start 77.18 108.81) (end 15.36 46.99) (width 0.8) (layer "F.Cu") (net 1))
 (segment (start 104.45 172.72) (end 104.45 170.035) (width 0.8) (layer "F.Cu") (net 1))
 (segment (start 77.18 142.765) (end 77.18 108.81) (width 0.8) (layer "F.Cu") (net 1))
 (segment (start 106.99 169.4) (end 79.085 141.495) (width 0.8) (layer "F.Cu") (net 8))
 (segment (start 35.905 64.025) (end 35.905 47.335) (width 0.8) (layer "F.Cu") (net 8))
 (segment (start 106.99 172.72) (end 106.99 169.4) (width 0.8) (layer "F.Cu") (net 8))
 (segment (start 79.085 107.205) (end 35.905 64.025) (width 0.8) (layer "F.Cu") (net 8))
 (segment (start 79.085 141.495) (end 79.085 107.205) (width 0.8) (layer "F.Cu") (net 8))
 (segment (start 35.905 47.335) (end 35.56 46.99) (width 0.8) (layer "F.Cu") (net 8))
 (segment (start 55.87 80.18) (end 55.87 47.1) (width 0.8) (layer "F.Cu") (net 4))
 (segment (start 109.53 169.4) (end 80.99 140.86) (width 0.8) (layer "F.Cu") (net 4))
 (segment (start 80.99 140.86) (end 80.99 105.3) (width 0.8) (layer "F.Cu") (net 4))
 (segment (start 55.87 47.1) (end 55.76 46.99) (width 0.8) (layer "F.Cu") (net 4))
 (segment (start 80.99 105.3) (end 55.87 80.18) (width 0.8) (layer "F.Cu") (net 4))
 (segment (start 109.53 172.72) (end 109.53 169.4) (width 0.8) (layer "F.Cu") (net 4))
 (segment (start 112.07 168.765) (end 82.895 139.59) (width 0.8) (layer "F.Cu") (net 5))
 (segment (start 82.895 139.59) (end 82.895 53.925) (width 0.8) (layer "F.Cu") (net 5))
 (segment (start 112.07 172.72) (end 112.07 168.765) (width 0.8) (layer "F.Cu") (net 5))
 (segment (start 82.895 53.925) (end 75.96 46.99) (width 0.8) (layer "F.Cu") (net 5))
 (segment (start 97.2 48.03) (end 97.2 151.464578) (width 0.8) (layer "F.Cu") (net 6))
 (segment (start 116.325978 170.480978) (end 117.15 171.305) (width 0.8) (layer "F.Cu") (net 6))
 (segment (start 96.16 46.99) (end 97.2 48.03) (width 0.8) (layer "F.Cu") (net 6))
 (segment (start 117.15 171.305) (end 117.15 172.72) (width 0.8) (layer "F.Cu") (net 6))
 (segment (start 97.2 151.464578) (end 116.2164 170.480978) (width 0.8) (layer "F.Cu") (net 6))
 (segment (start 116.2164 170.480978) (end 116.325978 170.480978) (width 0.8) (layer "F.Cu") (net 6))
 (segment (start 117.135327 58.994673) (end 103.215 72.915) (width 0.8) (layer "F.Cu") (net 7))
 (segment (start 103.215 154.939578) (end 118.7564 170.480978) (width 0.8) (layer "F.Cu") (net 7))
 (segment (start 117.135327 47.765327) (end 117.135327 58.994673) (width 0.8) (layer "F.Cu") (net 7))
 (segment (start 119.69 171.305) (end 119.69 172.72) (width 0.8) (layer "F.Cu") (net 7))
 (segment (start 103.215 72.915) (end 103.215 154.939578) (width 0.8) (layer "F.Cu") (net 7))
 (segment (start 118.865978 170.480978) (end 119.69 171.305) (width 0.8) (layer "F.Cu") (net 7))
 (segment (start 118.7564 170.480978) (end 118.865978 170.480978) (width 0.8) (layer "F.Cu") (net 7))
 (segment (start 116.36 46.99) (end 117.135327 47.765327) (width 0.8) (layer "F.Cu") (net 7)))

